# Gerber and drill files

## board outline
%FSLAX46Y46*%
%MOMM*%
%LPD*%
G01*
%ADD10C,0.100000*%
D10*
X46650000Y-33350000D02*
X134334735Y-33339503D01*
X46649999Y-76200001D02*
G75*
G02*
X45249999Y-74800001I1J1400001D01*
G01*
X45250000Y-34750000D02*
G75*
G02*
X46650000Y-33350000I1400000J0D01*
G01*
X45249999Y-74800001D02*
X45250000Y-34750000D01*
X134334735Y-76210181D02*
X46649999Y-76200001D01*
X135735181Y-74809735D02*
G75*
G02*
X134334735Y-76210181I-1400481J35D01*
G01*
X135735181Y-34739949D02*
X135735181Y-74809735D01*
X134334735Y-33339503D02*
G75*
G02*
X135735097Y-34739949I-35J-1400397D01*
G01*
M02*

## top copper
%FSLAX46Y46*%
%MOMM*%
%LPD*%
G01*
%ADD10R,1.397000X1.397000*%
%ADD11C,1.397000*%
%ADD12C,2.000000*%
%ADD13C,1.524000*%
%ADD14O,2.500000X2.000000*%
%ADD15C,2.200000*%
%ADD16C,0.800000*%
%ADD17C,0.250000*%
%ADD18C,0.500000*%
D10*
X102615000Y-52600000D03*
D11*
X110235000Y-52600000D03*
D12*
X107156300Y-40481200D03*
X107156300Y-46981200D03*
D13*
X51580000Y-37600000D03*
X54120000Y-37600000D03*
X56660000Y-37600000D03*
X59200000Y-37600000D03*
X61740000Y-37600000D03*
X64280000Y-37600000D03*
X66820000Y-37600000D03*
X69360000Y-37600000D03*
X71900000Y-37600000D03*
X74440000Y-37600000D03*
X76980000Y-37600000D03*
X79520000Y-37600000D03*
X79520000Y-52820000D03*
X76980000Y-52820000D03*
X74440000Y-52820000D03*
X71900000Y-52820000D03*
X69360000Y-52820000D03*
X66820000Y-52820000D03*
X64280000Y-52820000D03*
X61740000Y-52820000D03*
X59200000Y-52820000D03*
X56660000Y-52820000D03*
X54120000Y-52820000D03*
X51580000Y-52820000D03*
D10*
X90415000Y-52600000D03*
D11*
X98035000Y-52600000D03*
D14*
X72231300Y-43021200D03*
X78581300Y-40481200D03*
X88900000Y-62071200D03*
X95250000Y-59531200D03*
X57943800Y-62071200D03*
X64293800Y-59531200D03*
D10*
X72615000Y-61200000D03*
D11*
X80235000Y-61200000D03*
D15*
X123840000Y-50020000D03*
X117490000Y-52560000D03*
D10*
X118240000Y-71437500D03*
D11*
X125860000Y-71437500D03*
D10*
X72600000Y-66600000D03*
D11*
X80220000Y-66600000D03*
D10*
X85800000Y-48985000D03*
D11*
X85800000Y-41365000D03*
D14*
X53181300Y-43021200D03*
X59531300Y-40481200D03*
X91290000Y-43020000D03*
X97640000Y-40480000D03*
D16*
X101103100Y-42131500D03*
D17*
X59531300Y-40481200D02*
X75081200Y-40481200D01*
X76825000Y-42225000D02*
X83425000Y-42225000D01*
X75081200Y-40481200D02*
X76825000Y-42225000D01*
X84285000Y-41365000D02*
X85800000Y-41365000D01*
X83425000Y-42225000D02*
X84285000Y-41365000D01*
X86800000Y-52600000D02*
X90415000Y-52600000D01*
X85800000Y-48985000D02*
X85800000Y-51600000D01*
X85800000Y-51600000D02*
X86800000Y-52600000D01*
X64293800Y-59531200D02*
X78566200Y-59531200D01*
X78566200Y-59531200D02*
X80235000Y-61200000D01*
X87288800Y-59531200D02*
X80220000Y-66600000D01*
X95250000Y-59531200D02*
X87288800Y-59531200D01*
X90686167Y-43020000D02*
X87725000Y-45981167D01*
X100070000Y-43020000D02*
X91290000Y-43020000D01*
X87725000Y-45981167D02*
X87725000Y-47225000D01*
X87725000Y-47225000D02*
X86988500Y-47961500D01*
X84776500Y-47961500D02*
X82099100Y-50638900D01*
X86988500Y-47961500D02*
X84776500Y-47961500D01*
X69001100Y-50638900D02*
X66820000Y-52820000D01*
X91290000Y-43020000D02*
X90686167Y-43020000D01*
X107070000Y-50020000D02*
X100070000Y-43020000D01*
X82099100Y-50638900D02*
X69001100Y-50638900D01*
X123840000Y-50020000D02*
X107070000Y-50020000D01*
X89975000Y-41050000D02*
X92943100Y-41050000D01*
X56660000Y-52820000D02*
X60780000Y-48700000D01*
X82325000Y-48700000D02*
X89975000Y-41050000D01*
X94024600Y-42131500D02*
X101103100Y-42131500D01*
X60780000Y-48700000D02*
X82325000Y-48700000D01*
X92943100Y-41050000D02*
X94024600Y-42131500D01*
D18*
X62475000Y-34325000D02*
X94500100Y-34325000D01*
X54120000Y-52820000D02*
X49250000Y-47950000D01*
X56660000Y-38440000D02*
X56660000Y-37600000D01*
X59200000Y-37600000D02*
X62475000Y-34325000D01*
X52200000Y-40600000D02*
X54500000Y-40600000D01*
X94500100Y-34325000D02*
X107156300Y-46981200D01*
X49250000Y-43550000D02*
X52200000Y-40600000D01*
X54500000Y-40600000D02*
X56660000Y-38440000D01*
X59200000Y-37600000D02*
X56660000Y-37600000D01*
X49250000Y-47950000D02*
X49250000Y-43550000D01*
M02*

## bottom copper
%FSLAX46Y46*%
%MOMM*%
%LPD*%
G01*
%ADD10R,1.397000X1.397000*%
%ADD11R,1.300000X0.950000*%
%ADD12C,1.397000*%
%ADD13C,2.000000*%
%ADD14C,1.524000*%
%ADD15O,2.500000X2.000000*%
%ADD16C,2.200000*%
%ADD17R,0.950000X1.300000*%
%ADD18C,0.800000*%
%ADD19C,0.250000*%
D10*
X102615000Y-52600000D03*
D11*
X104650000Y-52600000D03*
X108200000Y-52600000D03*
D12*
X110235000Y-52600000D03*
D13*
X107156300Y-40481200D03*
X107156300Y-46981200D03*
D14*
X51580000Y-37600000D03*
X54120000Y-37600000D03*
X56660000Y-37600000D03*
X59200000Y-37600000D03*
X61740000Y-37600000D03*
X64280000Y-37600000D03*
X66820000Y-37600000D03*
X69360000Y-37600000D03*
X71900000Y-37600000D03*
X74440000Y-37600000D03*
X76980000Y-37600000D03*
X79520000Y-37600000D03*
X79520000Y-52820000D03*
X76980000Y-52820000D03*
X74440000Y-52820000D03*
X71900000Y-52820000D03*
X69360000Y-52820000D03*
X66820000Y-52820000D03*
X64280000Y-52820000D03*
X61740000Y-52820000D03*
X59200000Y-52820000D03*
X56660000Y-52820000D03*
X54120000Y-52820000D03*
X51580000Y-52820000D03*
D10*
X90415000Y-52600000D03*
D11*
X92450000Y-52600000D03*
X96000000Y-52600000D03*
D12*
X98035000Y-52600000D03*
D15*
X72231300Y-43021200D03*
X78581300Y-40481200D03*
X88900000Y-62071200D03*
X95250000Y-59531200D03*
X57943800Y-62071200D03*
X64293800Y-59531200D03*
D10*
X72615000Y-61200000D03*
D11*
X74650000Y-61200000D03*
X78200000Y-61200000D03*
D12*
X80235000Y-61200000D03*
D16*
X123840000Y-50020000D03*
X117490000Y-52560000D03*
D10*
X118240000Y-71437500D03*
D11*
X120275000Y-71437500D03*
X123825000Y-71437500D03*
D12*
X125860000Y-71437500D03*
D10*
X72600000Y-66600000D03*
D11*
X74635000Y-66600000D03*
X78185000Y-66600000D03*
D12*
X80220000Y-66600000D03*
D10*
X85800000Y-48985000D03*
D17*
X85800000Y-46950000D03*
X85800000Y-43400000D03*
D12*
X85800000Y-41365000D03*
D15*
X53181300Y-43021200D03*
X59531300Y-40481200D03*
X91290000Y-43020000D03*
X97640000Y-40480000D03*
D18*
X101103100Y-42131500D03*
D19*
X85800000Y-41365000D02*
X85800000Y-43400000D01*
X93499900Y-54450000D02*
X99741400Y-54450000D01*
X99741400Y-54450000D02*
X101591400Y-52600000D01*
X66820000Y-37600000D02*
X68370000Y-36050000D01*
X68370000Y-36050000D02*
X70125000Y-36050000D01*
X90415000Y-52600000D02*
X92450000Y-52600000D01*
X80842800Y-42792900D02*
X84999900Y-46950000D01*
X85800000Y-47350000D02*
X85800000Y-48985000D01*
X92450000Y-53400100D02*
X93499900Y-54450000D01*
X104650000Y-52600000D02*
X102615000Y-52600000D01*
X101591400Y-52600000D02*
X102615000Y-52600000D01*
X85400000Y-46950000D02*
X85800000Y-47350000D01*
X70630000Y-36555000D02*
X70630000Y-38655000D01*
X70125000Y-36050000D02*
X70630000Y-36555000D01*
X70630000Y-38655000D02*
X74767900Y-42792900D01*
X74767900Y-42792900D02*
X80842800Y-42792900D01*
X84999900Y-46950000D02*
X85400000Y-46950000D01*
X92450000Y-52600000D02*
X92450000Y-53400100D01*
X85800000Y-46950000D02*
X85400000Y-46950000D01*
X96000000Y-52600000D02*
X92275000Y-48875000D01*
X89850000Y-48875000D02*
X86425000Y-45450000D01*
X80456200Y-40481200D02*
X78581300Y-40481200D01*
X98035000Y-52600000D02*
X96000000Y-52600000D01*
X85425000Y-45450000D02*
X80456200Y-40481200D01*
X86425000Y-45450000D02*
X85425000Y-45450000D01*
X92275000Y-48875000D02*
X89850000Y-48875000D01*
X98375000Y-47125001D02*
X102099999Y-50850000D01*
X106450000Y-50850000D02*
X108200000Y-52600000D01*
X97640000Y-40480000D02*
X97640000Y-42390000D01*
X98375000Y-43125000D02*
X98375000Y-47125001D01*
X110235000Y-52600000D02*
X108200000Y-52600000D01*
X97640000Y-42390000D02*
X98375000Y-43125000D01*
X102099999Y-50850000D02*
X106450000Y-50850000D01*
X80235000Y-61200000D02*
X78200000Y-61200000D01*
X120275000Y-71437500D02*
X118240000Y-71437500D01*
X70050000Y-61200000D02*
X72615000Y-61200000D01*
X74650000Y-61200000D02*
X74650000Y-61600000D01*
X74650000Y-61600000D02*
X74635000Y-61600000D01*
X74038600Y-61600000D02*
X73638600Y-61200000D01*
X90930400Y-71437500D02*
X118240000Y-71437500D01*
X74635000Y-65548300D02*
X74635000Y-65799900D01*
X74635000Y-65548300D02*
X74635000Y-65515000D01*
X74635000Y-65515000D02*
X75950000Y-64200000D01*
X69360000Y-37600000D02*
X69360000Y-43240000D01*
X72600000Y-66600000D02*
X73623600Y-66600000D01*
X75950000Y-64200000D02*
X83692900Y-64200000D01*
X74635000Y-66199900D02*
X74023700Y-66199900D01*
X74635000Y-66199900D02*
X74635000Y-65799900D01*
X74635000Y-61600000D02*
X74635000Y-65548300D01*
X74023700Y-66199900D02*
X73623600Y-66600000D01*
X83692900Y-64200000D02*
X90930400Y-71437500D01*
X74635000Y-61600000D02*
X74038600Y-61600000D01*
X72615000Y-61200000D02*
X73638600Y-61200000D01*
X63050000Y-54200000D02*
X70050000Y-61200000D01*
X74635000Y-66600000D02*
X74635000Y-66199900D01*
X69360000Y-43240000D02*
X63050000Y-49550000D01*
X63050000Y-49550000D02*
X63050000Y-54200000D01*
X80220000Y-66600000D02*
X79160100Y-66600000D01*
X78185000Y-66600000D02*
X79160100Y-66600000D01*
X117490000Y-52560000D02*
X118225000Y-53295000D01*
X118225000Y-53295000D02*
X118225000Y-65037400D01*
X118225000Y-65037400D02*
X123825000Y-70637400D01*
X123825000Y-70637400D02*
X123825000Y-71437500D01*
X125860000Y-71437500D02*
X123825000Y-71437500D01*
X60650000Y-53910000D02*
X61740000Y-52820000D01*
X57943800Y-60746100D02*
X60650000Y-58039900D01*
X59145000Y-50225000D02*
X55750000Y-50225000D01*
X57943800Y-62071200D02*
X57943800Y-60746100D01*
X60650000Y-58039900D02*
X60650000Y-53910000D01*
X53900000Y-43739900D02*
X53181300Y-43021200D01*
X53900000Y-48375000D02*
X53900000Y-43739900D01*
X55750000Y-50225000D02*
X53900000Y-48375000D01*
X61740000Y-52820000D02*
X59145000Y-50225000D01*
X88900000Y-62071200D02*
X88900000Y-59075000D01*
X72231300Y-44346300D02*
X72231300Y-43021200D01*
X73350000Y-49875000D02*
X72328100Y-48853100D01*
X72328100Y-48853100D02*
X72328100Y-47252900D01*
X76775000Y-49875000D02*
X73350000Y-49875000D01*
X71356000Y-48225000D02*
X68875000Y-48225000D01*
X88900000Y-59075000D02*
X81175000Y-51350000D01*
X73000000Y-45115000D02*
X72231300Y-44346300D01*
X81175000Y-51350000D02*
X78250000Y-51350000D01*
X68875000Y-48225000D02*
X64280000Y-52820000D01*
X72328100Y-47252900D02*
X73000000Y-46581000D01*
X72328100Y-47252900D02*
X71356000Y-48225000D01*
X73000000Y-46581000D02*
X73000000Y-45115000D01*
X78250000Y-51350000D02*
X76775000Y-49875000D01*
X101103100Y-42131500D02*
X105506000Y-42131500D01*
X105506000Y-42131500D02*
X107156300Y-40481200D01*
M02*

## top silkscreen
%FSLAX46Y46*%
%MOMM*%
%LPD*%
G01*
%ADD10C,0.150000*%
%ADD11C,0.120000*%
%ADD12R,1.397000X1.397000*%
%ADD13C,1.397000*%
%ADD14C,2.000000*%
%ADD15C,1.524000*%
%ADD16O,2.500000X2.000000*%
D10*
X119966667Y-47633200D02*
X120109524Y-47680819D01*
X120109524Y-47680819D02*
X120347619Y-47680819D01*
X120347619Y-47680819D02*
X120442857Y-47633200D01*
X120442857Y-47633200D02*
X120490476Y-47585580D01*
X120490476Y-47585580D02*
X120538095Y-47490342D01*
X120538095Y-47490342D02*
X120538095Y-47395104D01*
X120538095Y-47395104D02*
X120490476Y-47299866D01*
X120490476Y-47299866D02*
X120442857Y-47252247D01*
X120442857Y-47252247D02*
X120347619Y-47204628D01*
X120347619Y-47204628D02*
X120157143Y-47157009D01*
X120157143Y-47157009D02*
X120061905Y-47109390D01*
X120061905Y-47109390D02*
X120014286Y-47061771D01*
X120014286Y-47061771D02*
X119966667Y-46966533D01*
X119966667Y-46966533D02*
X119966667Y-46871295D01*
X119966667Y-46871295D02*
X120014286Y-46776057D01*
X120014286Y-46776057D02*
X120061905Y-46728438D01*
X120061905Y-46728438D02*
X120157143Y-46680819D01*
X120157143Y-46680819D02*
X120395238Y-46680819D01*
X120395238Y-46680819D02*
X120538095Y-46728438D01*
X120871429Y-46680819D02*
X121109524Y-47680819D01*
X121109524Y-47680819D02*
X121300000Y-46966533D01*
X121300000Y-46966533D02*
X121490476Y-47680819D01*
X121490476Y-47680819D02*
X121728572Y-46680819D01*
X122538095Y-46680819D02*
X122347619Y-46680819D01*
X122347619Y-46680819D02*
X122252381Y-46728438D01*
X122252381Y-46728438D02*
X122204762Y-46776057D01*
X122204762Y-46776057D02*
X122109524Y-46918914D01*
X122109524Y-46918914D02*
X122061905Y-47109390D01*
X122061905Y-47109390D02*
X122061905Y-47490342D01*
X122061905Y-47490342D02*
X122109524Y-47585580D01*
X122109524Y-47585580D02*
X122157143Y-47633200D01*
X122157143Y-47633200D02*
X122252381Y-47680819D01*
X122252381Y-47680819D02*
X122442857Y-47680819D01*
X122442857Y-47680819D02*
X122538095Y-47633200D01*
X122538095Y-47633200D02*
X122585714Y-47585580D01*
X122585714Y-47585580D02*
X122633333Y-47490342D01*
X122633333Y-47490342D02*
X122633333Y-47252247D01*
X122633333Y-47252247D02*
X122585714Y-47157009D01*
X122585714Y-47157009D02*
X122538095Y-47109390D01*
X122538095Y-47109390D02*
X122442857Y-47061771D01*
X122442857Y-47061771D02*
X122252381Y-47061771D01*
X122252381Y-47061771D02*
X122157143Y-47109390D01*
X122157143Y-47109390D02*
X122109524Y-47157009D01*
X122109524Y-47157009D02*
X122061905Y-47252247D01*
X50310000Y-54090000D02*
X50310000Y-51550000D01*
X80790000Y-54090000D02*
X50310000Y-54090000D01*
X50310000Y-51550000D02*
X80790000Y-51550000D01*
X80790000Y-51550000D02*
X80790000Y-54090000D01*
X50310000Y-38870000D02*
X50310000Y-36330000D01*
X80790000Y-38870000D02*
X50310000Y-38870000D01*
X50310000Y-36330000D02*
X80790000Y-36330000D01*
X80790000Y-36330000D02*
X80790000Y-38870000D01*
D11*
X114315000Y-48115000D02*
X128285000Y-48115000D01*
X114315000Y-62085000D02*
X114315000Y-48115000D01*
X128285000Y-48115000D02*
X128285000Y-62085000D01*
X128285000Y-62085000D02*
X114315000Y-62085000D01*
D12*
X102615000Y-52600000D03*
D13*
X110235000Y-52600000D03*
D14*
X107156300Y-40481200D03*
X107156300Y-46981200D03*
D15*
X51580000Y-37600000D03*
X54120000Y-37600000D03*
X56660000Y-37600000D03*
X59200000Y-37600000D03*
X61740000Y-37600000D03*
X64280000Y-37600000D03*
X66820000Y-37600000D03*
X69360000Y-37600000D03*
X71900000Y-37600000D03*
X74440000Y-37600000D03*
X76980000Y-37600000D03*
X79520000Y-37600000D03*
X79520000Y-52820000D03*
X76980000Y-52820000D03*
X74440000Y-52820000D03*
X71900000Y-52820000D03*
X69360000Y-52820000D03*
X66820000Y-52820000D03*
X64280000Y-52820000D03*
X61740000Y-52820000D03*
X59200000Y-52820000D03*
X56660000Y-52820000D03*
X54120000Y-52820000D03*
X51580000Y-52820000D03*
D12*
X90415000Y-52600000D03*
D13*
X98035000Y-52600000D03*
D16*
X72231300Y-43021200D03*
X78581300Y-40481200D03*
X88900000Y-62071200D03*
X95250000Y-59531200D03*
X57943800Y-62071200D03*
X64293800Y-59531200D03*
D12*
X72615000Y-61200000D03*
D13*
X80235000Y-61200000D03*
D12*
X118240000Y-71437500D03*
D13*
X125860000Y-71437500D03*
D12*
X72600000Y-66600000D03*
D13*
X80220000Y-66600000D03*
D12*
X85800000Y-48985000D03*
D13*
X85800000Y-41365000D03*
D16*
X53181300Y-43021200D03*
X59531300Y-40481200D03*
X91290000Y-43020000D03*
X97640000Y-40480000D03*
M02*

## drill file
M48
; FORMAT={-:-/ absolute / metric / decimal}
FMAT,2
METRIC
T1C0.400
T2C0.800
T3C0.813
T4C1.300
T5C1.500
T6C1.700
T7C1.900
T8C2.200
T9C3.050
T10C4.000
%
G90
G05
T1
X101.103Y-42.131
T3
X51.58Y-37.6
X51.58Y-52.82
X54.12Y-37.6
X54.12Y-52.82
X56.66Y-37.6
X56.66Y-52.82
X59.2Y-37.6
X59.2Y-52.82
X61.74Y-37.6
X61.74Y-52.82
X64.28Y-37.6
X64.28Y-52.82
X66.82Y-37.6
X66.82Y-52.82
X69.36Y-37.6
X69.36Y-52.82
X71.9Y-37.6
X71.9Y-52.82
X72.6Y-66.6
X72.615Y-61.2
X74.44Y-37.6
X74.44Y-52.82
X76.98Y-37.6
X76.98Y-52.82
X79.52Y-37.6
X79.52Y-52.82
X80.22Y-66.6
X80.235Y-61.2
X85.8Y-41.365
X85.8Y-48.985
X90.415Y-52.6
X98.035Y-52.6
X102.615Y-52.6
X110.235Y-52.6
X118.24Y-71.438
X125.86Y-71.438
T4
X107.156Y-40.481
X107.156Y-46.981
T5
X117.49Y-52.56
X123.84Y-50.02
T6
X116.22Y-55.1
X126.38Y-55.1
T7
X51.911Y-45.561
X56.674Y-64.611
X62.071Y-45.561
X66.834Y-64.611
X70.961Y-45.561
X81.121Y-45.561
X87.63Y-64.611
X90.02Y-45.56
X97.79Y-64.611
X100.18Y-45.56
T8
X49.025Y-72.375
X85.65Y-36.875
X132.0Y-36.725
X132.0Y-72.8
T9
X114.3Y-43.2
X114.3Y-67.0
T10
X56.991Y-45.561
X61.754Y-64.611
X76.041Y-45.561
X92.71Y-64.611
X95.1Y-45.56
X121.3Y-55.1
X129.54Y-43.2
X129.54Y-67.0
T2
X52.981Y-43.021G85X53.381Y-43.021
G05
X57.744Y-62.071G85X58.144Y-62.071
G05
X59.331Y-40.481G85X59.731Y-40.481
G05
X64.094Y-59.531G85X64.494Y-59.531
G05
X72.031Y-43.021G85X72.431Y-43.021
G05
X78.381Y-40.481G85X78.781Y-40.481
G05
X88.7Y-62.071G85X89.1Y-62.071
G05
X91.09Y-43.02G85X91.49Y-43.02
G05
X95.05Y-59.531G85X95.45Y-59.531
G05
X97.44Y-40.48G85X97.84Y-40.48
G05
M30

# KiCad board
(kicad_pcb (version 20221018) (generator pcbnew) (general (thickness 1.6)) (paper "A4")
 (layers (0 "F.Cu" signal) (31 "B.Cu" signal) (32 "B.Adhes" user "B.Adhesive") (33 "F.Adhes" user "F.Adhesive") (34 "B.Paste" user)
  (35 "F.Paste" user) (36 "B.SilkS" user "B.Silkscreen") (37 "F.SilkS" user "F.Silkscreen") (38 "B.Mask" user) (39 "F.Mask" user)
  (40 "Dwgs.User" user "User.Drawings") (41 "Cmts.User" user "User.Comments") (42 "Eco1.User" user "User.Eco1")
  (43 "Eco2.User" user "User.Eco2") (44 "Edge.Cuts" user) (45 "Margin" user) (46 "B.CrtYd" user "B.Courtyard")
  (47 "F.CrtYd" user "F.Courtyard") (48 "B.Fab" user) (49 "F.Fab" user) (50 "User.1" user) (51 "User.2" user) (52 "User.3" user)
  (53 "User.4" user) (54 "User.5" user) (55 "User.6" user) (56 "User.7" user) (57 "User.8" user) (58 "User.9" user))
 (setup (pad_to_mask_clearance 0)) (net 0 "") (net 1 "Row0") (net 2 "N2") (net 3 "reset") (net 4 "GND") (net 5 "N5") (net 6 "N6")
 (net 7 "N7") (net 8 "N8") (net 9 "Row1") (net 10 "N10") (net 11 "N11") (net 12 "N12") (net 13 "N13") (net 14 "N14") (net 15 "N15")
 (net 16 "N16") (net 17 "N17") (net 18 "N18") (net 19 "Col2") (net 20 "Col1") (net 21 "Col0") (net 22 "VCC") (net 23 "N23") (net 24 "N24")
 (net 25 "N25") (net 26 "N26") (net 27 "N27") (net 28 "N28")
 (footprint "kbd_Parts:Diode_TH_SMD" (layer "F.Cu") (at 106.425 52.6)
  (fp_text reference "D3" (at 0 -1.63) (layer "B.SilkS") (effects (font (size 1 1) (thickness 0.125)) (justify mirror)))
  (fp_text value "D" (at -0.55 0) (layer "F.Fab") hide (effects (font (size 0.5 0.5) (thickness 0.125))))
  (pad "1" thru_hole rect (at -3.81 0) (size 1.397 1.397) (drill 0.8128) (layers "*.Cu" "*.Mask" "F.SilkS") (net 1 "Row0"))
  (pad "1" smd rect (at -1.775 0) (size 1.3 0.95) (layers "B.Cu" "B.Paste" "B.Mask") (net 1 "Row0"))
  (pad "2" smd rect (at 1.775 0) (size 1.3 0.95) (layers "B.Cu" "B.Paste" "B.Mask") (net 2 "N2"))
  (pad "2" thru_hole circle (at 3.81 0) (size 1.397 1.397) (drill 0.8128) (layers "*.Cu" "*.Mask" "F.SilkS") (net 2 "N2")))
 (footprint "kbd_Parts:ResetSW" (layer "F.Cu") (at 107.1563 43.7312 90)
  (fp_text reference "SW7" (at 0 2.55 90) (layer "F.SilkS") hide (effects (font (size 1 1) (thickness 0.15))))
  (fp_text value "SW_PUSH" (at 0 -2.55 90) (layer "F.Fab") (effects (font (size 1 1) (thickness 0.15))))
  (pad "1" thru_hole circle (at 3.25 0 90) (size 2 2) (drill 1.3) (layers "*.Cu" "*.Mask" "F.SilkS") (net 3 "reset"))
  (pad "2" thru_hole circle (at -3.25 0 90) (size 2 2) (drill 1.3) (layers "*.Cu" "*.Mask" "F.SilkS") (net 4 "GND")))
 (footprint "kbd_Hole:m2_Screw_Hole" (layer "F.Cu") (at 85.65 36.875)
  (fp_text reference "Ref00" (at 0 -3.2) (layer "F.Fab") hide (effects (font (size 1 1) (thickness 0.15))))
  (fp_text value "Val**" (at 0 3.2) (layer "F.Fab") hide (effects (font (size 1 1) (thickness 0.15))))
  (pad "" np_thru_hole circle (at 0 0) (size 2.2 2.2) (drill 2.2) (layers "*.Cu" "*.Mask")))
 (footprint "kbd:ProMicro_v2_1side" (layer "F.Cu") (at 66.058 45.2564 90)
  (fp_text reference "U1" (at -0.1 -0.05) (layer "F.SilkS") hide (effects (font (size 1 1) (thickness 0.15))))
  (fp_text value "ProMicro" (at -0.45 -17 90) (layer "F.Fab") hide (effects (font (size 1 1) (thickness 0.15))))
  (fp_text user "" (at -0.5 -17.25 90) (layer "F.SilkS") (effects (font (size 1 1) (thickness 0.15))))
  (fp_line (start -8.8336 -15.748) (end -6.2936 -15.748) (stroke (width 0.15) (type solid)) (layer "F.SilkS"))
  (fp_line (start -8.8336 14.732) (end -8.8336 -15.748) (stroke (width 0.15) (type solid)) (layer "F.SilkS"))
  (fp_line (start -6.2936 -15.748) (end -6.2936 14.732) (stroke (width 0.15) (type solid)) (layer "F.SilkS"))
  (fp_line (start -6.2936 14.732) (end -8.8336 14.732) (stroke (width 0.15) (type solid)) (layer "F.SilkS"))
  (fp_line (start 6.3864 -15.748) (end 8.9264 -15.748) (stroke (width 0.15) (type solid)) (layer "F.SilkS"))
  (fp_line (start 6.3864 14.732) (end 6.3864 -15.748) (stroke (width 0.15) (type solid)) (layer "F.SilkS"))
  (fp_line (start 8.9264 -15.748) (end 8.9264 14.732) (stroke (width 0.15) (type solid)) (layer "F.SilkS"))
  (fp_line (start 8.9264 14.732) (end 6.3864 14.732) (stroke (width 0.15) (type solid)) (layer "F.SilkS"))
  (pad "1" thru_hole circle (at 7.6564 -14.478 90) (size 1.524 1.524) (drill 0.8128) (layers "*.Cu" "F.SilkS" "B.Mask") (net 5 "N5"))
  (pad "2" thru_hole circle (at 7.6564 -11.938 90) (size 1.524 1.524) (drill 0.8128) (layers "*.Cu" "F.SilkS" "B.Mask") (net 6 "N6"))
  (pad "3" thru_hole circle (at 7.6564 -9.398 90) (size 1.524 1.524) (drill 0.8128) (layers "*.Cu" "F.SilkS" "B.Mask") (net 4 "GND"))
  (pad "4" thru_hole circle (at 7.6564 -6.858 90) (size 1.524 1.524) (drill 0.8128) (layers "*.Cu" "F.SilkS" "B.Mask") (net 4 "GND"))
  (pad "5" thru_hole circle (at 7.6564 -4.318 90) (size 1.524 1.524) (drill 0.8128) (layers "*.Cu" "F.SilkS" "B.Mask") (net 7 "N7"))
  (pad "6" thru_hole circle (at 7.6564 -1.778 90) (size 1.524 1.524) (drill 0.8128) (layers "*.Cu" "F.SilkS" "B.Mask") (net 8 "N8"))
  (pad "7" thru_hole circle (at 7.6564 0.762 90) (size 1.524 1.524) (drill 0.8128) (layers "*.Cu" "F.SilkS" "B.Mask") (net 1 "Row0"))
  (pad "8" thru_hole circle (at 7.6564 3.302 90) (size 1.524 1.524) (drill 0.8128) (layers "*.Cu" "F.SilkS" "B.Mask") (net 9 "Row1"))
  (pad "9" thru_hole circle (at 7.6564 5.842 90) (size 1.524 1.524) (drill 0.8128) (layers "*.Cu" "F.SilkS" "B.Mask") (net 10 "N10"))
  (pad "10" thru_hole circle (at 7.6564 8.382 90) (size 1.524 1.524) (drill 0.8128) (layers "*.Cu" "F.SilkS" "B.Mask") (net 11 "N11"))
  (pad "11" thru_hole circle (at 7.6564 10.922 90) (size 1.524 1.524) (drill 0.8128) (layers "*.Cu" "F.SilkS" "B.Mask") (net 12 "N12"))
  (pad "12" thru_hole circle (at 7.6564 13.462 90) (size 1.524 1.524) (drill 0.8128) (layers "*.Cu" "F.SilkS" "B.Mask") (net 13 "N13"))
  (pad "13" thru_hole circle (at -7.5636 13.462 90) (size 1.524 1.524) (drill 0.8128) (layers "*.Cu" "F.SilkS" "B.Mask") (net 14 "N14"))
  (pad "14" thru_hole circle (at -7.5636 10.922 90) (size 1.524 1.524) (drill 0.8128) (layers "*.Cu" "F.SilkS" "B.Mask") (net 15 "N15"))
  (pad "15" thru_hole circle (at -7.5636 8.382 90) (size 1.524 1.524) (drill 0.8128) (layers "*.Cu" "F.SilkS" "B.Mask") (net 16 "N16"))
  (pad "16" thru_hole circle (at -7.5636 5.842 90) (size 1.524 1.524) (drill 0.8128) (layers "*.Cu" "F.SilkS" "B.Mask") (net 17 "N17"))
  (pad "17" thru_hole circle (at -7.5636 3.302 90) (size 1.524 1.524) (drill 0.8128) (layers "*.Cu" "F.SilkS" "B.Mask") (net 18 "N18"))
  (pad "18" thru_hole circle (at -7.5636 0.762 90) (size 1.524 1.524) (drill 0.8128) (layers "*.Cu" "F.SilkS" "B.Mask") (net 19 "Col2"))
  (pad "19" thru_hole circle (at -7.5636 -1.778 90) (size 1.524 1.524) (drill 0.8128) (layers "*.Cu" "F.SilkS" "B.Mask") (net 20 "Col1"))
  (pad "20" thru_hole circle (at -7.5636 -4.318 90) (size 1.524 1.524) (drill 0.8128) (layers "*.Cu" "F.SilkS" "B.Mask") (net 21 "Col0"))
  (pad "21" thru_hole circle (at -7.5636 -6.858 90) (size 1.524 1.524) (drill 0.8128) (layers "*.Cu" "F.SilkS" "B.Mask") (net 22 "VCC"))
  (pad "22" thru_hole circle (at -7.5636 -9.398 90) (size 1.524 1.524) (drill 0.8128) (layers "*.Cu" "F.SilkS" "B.Mask") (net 3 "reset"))
  (pad "23" thru_hole circle (at -7.5636 -11.938 90) (size 1.524 1.524) (drill 0.8128) (layers "*.Cu" "F.SilkS" "B.Mask") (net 4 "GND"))
  (pad "24" thru_hole circle (at -7.5636 -14.478 90) (size 1.524 1.524) (drill 0.8128) (layers "*.Cu" "F.SilkS" "B.Mask") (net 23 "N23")))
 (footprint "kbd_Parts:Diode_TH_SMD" (layer "F.Cu") (at 94.225 52.6)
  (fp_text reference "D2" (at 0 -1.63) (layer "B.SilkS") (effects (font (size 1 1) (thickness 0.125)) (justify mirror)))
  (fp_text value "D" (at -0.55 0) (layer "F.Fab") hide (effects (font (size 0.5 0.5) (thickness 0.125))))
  (pad "1" thru_hole rect (at -3.81 0) (size 1.397 1.397) (drill 0.8128) (layers "*.Cu" "*.Mask" "F.SilkS") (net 1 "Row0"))
  (pad "1" smd rect (at -1.775 0) (size 1.3 0.95) (layers "B.Cu" "B.Paste" "B.Mask") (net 1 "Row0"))
  (pad "2" smd rect (at 1.775 0) (size 1.3 0.95) (layers "B.Cu" "B.Paste" "B.Mask") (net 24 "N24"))
  (pad "2" thru_hole circle (at 3.81 0) (size 1.397 1.397) (drill 0.8128) (layers "*.Cu" "*.Mask" "F.SilkS") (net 24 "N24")))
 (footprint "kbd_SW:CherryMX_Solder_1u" (layer "F.Cu") (at 76.0413 45.5612)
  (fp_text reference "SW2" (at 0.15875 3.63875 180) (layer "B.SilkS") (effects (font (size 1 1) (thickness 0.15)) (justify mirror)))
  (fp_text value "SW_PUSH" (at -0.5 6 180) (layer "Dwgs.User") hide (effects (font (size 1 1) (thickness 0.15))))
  (pad "" np_thru_hole circle (at -5.08 0 90) (size 1.9 1.9) (drill 1.9) (layers "*.Cu" "*.Mask"))
  (pad "" np_thru_hole circle (at 0 0 90) (size 4 4) (drill 4) (layers "*.Cu" "*.Mask"))
  (pad "" np_thru_hole circle (at 5.08 0 90) (size 1.9 1.9) (drill 1.9) (layers "*.Cu" "*.Mask"))
  (pad "1" thru_hole oval (at -3.81 -2.54) (size 2.5 2) (drill oval 1.2 0.8) (layers "*.Cu" "F.SilkS" "B.Mask") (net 20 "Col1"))
  (pad "2" thru_hole oval (at 2.54 -5.08) (size 2.5 2) (drill oval 1.2 0.8) (layers "*.Cu" "F.SilkS" "B.Mask") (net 24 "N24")))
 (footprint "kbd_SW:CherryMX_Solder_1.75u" (layer "F.Cu") (at 92.71 64.6112)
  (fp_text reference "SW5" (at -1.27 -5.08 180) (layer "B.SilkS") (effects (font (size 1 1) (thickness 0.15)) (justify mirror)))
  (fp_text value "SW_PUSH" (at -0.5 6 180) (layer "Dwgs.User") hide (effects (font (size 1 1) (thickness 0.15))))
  (pad "" np_thru_hole circle (at -5.08 0 90) (size 1.9 1.9) (drill 1.9) (layers "*.Cu" "*.Mask"))
  (pad "" np_thru_hole circle (at 0 0 90) (size 4 4) (drill 4) (layers "*.Cu" "*.Mask"))
  (pad "" np_thru_hole circle (at 5.08 0 90) (size 1.9 1.9) (drill 1.9) (layers "*.Cu" "*.Mask"))
  (pad "1" thru_hole oval (at -3.81 -2.54) (size 2.5 2) (drill oval 1.2 0.8) (layers "*.Cu" "F.SilkS" "B.Mask") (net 20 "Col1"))
  (pad "2" thru_hole oval (at 2.54 -5.08) (size 2.5 2) (drill oval 1.2 0.8) (layers "*.Cu" "F.SilkS" "B.Mask") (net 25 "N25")))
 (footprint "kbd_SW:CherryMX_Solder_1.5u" (layer "F.Cu") (at 61.7538 64.6112)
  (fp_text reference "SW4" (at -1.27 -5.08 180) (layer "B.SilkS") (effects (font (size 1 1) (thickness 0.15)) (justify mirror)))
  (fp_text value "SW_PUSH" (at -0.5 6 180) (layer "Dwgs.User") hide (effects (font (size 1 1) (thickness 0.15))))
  (pad "" np_thru_hole circle (at -5.08 0 90) (size 1.9 1.9) (drill 1.9) (layers "*.Cu" "*.Mask"))
  (pad "" np_thru_hole circle (at 0 0 90) (size 4 4) (drill 4) (layers "*.Cu" "*.Mask"))
  (pad "" np_thru_hole circle (at 5.08 0 90) (size 1.9 1.9) (drill 1.9) (layers "*.Cu" "*.Mask"))
  (pad "1" thru_hole oval (at -3.81 -2.54) (size 2.5 2) (drill oval 1.2 0.8) (layers "*.Cu" "F.SilkS" "B.Mask") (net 21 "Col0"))
  (pad "2" thru_hole oval (at 2.54 -5.08) (size 2.5 2) (drill oval 1.2 0.8) (layers "*.Cu" "F.SilkS" "B.Mask") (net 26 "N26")))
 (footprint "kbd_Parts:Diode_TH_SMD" (layer "F.Cu") (at 76.425 61.2)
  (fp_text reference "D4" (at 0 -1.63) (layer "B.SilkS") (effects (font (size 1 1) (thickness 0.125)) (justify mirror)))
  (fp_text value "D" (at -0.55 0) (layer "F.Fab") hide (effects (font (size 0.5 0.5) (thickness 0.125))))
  (pad "1" thru_hole rect (at -3.81 0) (size 1.397 1.397) (drill 0.8128) (layers "*.Cu" "*.Mask" "F.SilkS") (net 9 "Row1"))
  (pad "1" smd rect (at -1.775 0) (size 1.3 0.95) (layers "B.Cu" "B.Paste" "B.Mask") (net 9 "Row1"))
  (pad "2" smd rect (at 1.775 0) (size 1.3 0.95) (layers "B.Cu" "B.Paste" "B.Mask") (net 26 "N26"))
  (pad "2" thru_hole circle (at 3.81 0) (size 1.397 1.397) (drill 0.8128) (layers "*.Cu" "*.Mask" "F.SilkS") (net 26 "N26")))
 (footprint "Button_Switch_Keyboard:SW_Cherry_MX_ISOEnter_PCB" (layer "F.Cu") (at 123.84 50.02)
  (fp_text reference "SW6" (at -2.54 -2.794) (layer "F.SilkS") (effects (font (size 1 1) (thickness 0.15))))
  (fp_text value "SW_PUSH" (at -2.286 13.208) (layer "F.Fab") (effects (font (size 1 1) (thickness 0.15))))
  (fp_line (start -9.525 -1.905) (end 4.445 -1.905) (stroke (width 0.12) (type solid)) (layer "F.SilkS"))
  (fp_line (start -9.525 12.065) (end -9.525 -1.905) (stroke (width 0.12) (type solid)) (layer "F.SilkS"))
  (fp_line (start 4.445 -1.905) (end 4.445 12.065) (stroke (width 0.12) (type solid)) (layer "F.SilkS"))
  (fp_line (start 4.445 12.065) (end -9.525 12.065) (stroke (width 0.12) (type solid)) (layer "F.SilkS"))
  (pad "" np_thru_hole circle (at -9.54 -6.82) (size 3.05 3.05) (drill 3.05) (layers "*.Cu" "*.Mask"))
  (pad "" np_thru_hole circle (at -9.54 16.98) (size 3.05 3.05) (drill 3.05) (layers "*.Cu" "*.Mask"))
  (pad "" np_thru_hole circle (at -7.62 5.08) (size 1.7 1.7) (drill 1.7) (layers "*.Cu" "*.Mask"))
  (pad "" np_thru_hole circle (at -2.54 5.08) (size 4 4) (drill 4) (layers "*.Cu" "*.Mask"))
  (pad "" np_thru_hole circle (at 2.54 5.08) (size 1.7 1.7) (drill 1.7) (layers "*.Cu" "*.Mask"))
  (pad "" np_thru_hole circle (at 5.7 -6.82) (size 4 4) (drill 4) (layers "*.Cu" "*.Mask"))
  (pad "" np_thru_hole circle (at 5.7 16.98) (size 4 4) (drill 4) (layers "*.Cu" "*.Mask"))
  (pad "1" thru_hole circle (at 0 0) (size 2.2 2.2) (drill 1.5) (layers "*.Cu" "*.Mask") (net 19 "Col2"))
  (pad "2" thru_hole circle (at -6.35 2.54) (size 2.2 2.2) (drill 1.5) (layers "*.Cu" "*.Mask") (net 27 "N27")))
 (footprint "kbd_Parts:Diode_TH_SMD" (layer "F.Cu") (at 122.05 71.4375)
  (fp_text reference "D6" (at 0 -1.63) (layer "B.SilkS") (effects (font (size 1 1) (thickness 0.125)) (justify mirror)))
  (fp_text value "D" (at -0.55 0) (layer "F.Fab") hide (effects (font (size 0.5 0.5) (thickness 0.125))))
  (pad "1" thru_hole rect (at -3.81 0) (size 1.397 1.397) (drill 0.8128) (layers "*.Cu" "*.Mask" "F.SilkS") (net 9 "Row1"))
  (pad "1" smd rect (at -1.775 0) (size 1.3 0.95) (layers "B.Cu" "B.Paste" "B.Mask") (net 9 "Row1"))
  (pad "2" smd rect (at 1.775 0) (size 1.3 0.95) (layers "B.Cu" "B.Paste" "B.Mask") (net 27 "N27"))
  (pad "2" thru_hole circle (at 3.81 0) (size 1.397 1.397) (drill 0.8128) (layers "*.Cu" "*.Mask" "F.SilkS") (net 27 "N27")))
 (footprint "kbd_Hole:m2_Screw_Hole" (layer "F.Cu") (at 132 36.725)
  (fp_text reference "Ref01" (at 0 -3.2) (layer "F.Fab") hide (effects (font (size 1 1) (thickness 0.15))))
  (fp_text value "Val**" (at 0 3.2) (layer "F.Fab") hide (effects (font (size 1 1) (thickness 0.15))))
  (pad "" np_thru_hole circle (at 0 0) (size 2.2 2.2) (drill 2.2) (layers "*.Cu" "*.Mask")))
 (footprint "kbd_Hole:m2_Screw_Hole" (layer "F.Cu") (at 132 72.8)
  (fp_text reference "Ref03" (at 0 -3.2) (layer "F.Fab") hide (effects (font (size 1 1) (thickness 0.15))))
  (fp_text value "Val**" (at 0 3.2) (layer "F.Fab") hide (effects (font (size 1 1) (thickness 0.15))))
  (pad "" np_thru_hole circle (at 0 0) (size 2.2 2.2) (drill 2.2) (layers "*.Cu" "*.Mask")))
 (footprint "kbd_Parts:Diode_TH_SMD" (layer "F.Cu") (at 76.41 66.6)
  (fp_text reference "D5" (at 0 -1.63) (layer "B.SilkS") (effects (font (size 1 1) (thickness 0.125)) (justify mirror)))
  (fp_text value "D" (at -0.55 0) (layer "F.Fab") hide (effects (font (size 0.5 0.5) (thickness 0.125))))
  (pad "1" thru_hole rect (at -3.81 0) (size 1.397 1.397) (drill 0.8128) (layers "*.Cu" "*.Mask" "F.SilkS") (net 9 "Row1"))
  (pad "1" smd rect (at -1.775 0) (size 1.3 0.95) (layers "B.Cu" "B.Paste" "B.Mask") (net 9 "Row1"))
  (pad "2" smd rect (at 1.775 0) (size 1.3 0.95) (layers "B.Cu" "B.Paste" "B.Mask") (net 25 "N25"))
  (pad "2" thru_hole circle (at 3.81 0) (size 1.397 1.397) (drill 0.8128) (layers "*.Cu" "*.Mask" "F.SilkS") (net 25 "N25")))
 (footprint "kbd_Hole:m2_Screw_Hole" (layer "F.Cu") (at 49.025 72.375)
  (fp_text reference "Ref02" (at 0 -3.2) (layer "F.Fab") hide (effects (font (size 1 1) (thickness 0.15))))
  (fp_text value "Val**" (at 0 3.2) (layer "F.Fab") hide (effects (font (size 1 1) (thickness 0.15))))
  (pad "" np_thru_hole circle (at 0 0) (size 2.2 2.2) (drill 2.2) (layers "*.Cu" "*.Mask")))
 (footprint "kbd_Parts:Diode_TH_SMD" (layer "F.Cu") (at 85.8 45.175 90)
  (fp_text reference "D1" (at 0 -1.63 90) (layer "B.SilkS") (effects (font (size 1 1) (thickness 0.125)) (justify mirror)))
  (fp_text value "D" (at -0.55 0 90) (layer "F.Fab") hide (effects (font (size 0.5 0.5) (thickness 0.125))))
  (pad "1" thru_hole rect (at -3.81 0 90) (size 1.397 1.397) (drill 0.8128) (layers "*.Cu" "*.Mask" "F.SilkS") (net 1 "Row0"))
  (pad "1" smd rect (at -1.775 0 90) (size 1.3 0.95) (layers "B.Cu" "B.Paste" "B.Mask") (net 1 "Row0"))
  (pad "2" smd rect (at 1.775 0 90) (size 1.3 0.95) (layers "B.Cu" "B.Paste" "B.Mask") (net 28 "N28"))
  (pad "2" thru_hole circle (at 3.81 0 90) (size 1.397 1.397) (drill 0.8128) (layers "*.Cu" "*.Mask" "F.SilkS") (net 28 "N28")))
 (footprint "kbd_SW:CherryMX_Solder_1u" (layer "F.Cu") (at 56.9913 45.5612)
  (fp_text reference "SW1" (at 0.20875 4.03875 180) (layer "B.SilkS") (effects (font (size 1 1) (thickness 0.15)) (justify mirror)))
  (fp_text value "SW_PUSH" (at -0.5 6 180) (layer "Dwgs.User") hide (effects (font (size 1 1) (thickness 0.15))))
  (pad "" np_thru_hole circle (at -5.08 0 90) (size 1.9 1.9) (drill 1.9) (layers "*.Cu" "*.Mask"))
  (pad "" np_thru_hole circle (at 0 0 90) (size 4 4) (drill 4) (layers "*.Cu" "*.Mask"))
  (pad "" np_thru_hole circle (at 5.08 0 90) (size 1.9 1.9) (drill 1.9) (layers "*.Cu" "*.Mask"))
  (pad "1" thru_hole oval (at -3.81 -2.54) (size 2.5 2) (drill oval 1.2 0.8) (layers "*.Cu" "F.SilkS" "B.Mask") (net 21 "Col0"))
  (pad "2" thru_hole oval (at 2.54 -5.08) (size 2.5 2) (drill oval 1.2 0.8) (layers "*.Cu" "F.SilkS" "B.Mask") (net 28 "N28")))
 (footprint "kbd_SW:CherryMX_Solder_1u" (layer "F.Cu") (at 95.1 45.56)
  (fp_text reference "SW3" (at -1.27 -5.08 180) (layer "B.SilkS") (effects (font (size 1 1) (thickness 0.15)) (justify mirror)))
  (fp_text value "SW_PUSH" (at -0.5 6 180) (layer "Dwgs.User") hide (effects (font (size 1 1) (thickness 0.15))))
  (pad "" np_thru_hole circle (at -5.08 0 90) (size 1.9 1.9) (drill 1.9) (layers "*.Cu" "*.Mask"))
  (pad "" np_thru_hole circle (at 0 0 90) (size 4 4) (drill 4) (layers "*.Cu" "*.Mask"))
  (pad "" np_thru_hole circle (at 5.08 0 90) (size 1.9 1.9) (drill 1.9) (layers "*.Cu" "*.Mask"))
  (pad "1" thru_hole oval (at -3.81 -2.54) (size 2.5 2) (drill oval 1.2 0.8) (layers "*.Cu" "F.SilkS" "B.Mask") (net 19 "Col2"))
  (pad "2" thru_hole oval (at 2.54 -5.08) (size 2.5 2) (drill oval 1.2 0.8) (layers "*.Cu" "F.SilkS" "B.Mask") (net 2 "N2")))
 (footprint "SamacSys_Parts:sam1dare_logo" (layer "B.Cu") (at 105.4 69.4 180)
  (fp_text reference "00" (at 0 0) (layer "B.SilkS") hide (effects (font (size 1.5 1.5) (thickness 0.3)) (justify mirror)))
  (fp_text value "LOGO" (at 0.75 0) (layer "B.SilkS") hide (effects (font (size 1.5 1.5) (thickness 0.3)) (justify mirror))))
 (gr_line (start 46.65 33.35) (end 134.334735 33.339503) (stroke (width 0.1) (type default)) (layer "Edge.Cuts"))
 (gr_arc (start 46.649999 76.200001) (mid 45.66005 75.78995) (end 45.249999 74.800001) (stroke (width 0.1) (type default))
  (layer "Edge.Cuts"))
 (gr_arc (start 45.25 34.75) (mid 45.660051 33.760051) (end 46.65 33.35) (stroke (width 0.1) (type default)) (layer "Edge.Cuts"))
 (gr_line (start 45.249999 74.800001) (end 45.25 34.75) (stroke (width 0.1) (type default)) (layer "Edge.Cuts"))
 (gr_line (start 134.334735 76.210181) (end 46.649999 76.200001) (stroke (width 0.1) (type default)) (layer "Edge.Cuts"))
 (gr_arc (start 135.735181 74.809735) (mid 135.325 75.8) (end 134.334735 76.210181) (stroke (width 0.1) (type default)) (layer "Edge.Cuts"))
 (gr_line (start 135.735181 34.739949) (end 135.735181 74.809735) (stroke (width 0.1) (type default)) (layer "Edge.Cuts"))
 (gr_arc (start 134.334735 33.339503) (mid 135.325 33.749684) (end 135.735181 34.739949) (stroke (width 0.1) (type default))
  (layer "Edge.Cuts"))
 (segment (start 59.5313 40.4812) (end 75.0812 40.4812) (width 0.25) (layer "F.Cu") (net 28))
 (segment (start 76.825 42.225) (end 83.425 42.225) (width 0.25) (layer "F.Cu") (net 28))
 (segment (start 75.0812 40.4812) (end 76.825 42.225) (width 0.25) (layer "F.Cu") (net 28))
 (segment (start 84.285 41.365) (end 85.8 41.365) (width 0.25) (layer "F.Cu") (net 28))
 (segment (start 83.425 42.225) (end 84.285 41.365) (width 0.25) (layer "F.Cu") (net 28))
 (segment (start 85.8 41.365) (end 85.8 43.4) (width 0.25) (layer "B.Cu") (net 28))
 (segment (start 86.8 52.6) (end 90.415 52.6) (width 0.25) (layer "F.Cu") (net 1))
 (segment (start 85.8 48.985) (end 85.8 51.6) (width 0.25) (layer "F.Cu") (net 1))
 (segment (start 85.8 51.6) (end 86.8 52.6) (width 0.25) (layer "F.Cu") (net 1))
 (segment (start 93.4999 54.45) (end 99.7414 54.45) (width 0.25) (layer "B.Cu") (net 1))
 (segment (start 99.7414 54.45) (end 101.5914 52.6) (width 0.25) (layer "B.Cu") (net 1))
 (segment (start 66.82 37.6) (end 68.37 36.05) (width 0.25) (layer "B.Cu") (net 1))
 (segment (start 68.37 36.05) (end 70.125 36.05) (width 0.25) (layer "B.Cu") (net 1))
 (segment (start 90.415 52.6) (end 92.45 52.6) (width 0.25) (layer "B.Cu") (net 1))
 (segment (start 80.8428 42.7929) (end 84.9999 46.95) (width 0.25) (layer "B.Cu") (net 1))
 (segment (start 85.8 47.35) (end 85.8 48.985) (width 0.25) (layer "B.Cu") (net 1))
 (segment (start 92.45 53.4001) (end 93.4999 54.45) (width 0.25) (layer "B.Cu") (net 1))
 (segment (start 104.65 52.6) (end 102.615 52.6) (width 0.25) (layer "B.Cu") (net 1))
 (segment (start 101.5914 52.6) (end 102.615 52.6) (width 0.25) (layer "B.Cu") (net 1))
 (segment (start 85.4 46.95) (end 85.8 47.35) (width 0.25) (layer "B.Cu") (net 1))
 (segment (start 70.63 36.555) (end 70.63 38.655) (width 0.25) (layer "B.Cu") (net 1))
 (segment (start 70.125 36.05) (end 70.63 36.555) (width 0.25) (layer "B.Cu") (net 1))
 (segment (start 70.63 38.655) (end 74.7679 42.7929) (width 0.25) (layer "B.Cu") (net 1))
 (segment (start 74.7679 42.7929) (end 80.8428 42.7929) (width 0.25) (layer "B.Cu") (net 1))
 (segment (start 84.9999 46.95) (end 85.4 46.95) (width 0.25) (layer "B.Cu") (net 1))
 (segment (start 92.45 52.6) (end 92.45 53.4001) (width 0.25) (layer "B.Cu") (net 1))
 (segment (start 85.8 46.95) (end 85.4 46.95) (width 0.25) (layer "B.Cu") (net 1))
 (segment (start 96 52.6) (end 92.275 48.875) (width 0.25) (layer "B.Cu") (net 24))
 (segment (start 89.85 48.875) (end 86.425 45.45) (width 0.25) (layer "B.Cu") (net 24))
 (segment (start 80.4562 40.4812) (end 78.5813 40.4812) (width 0.25) (layer "B.Cu") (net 24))
 (segment (start 98.035 52.6) (end 96 52.6) (width 0.25) (layer "B.Cu") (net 24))
 (segment (start 85.425 45.45) (end 80.4562 40.4812) (width 0.25) (layer "B.Cu") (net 24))
 (segment (start 86.425 45.45) (end 85.425 45.45) (width 0.25) (layer "B.Cu") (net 24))
 (segment (start 92.275 48.875) (end 89.85 48.875) (width 0.25) (layer "B.Cu") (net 24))
 (segment (start 98.375 47.125001) (end 102.099999 50.85) (width 0.25) (layer "B.Cu") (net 2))
 (segment (start 106.45 50.85) (end 108.2 52.6) (width 0.25) (layer "B.Cu") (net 2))
 (segment (start 97.64 40.48) (end 97.64 42.39) (width 0.25) (layer "B.Cu") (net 2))
 (segment (start 98.375 43.125) (end 98.375 47.125001) (width 0.25) (layer "B.Cu") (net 2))
 (segment (start 110.235 52.6) (end 108.2 52.6) (width 0.25) (layer "B.Cu") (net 2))
 (segment (start 97.64 42.39) (end 98.375 43.125) (width 0.25) (layer "B.Cu") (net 2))
 (segment (start 102.099999 50.85) (end 106.45 50.85) (width 0.25) (layer "B.Cu") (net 2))
 (segment (start 64.2938 59.5312) (end 78.5662 59.5312) (width 0.25) (layer "F.Cu") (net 26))
 (segment (start 78.5662 59.5312) (end 80.235 61.2) (width 0.25) (layer "F.Cu") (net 26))
 (segment (start 80.235 61.2) (end 78.2 61.2) (width 0.25) (layer "B.Cu") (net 26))
 (segment (start 120.275 71.4375) (end 118.24 71.4375) (width 0.25) (layer "B.Cu") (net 9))
 (segment (start 70.05 61.2) (end 72.615 61.2) (width 0.25) (layer "B.Cu") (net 9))
 (segment (start 74.65 61.2) (end 74.65 61.6) (width 0.25) (layer "B.Cu") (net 9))
 (segment (start 74.65 61.6) (end 74.635 61.6) (width 0.25) (layer "B.Cu") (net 9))
 (segment (start 74.0386 61.6) (end 73.6386 61.2) (width 0.25) (layer "B.Cu") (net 9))
 (segment (start 90.9304 71.4375) (end 118.24 71.4375) (width 0.25) (layer "B.Cu") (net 9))
 (segment (start 74.635 65.5483) (end 74.635 65.7999) (width 0.25) (layer "B.Cu") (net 9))
 (segment (start 74.635 65.5483) (end 74.635 65.515) (width 0.25) (layer "B.Cu") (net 9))
 (segment (start 74.635 65.515) (end 75.95 64.2) (width 0.25) (layer "B.Cu") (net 9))
 (segment (start 69.36 37.6) (end 69.36 43.24) (width 0.25) (layer "B.Cu") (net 9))
 (segment (start 72.6 66.6) (end 73.6236 66.6) (width 0.25) (layer "B.Cu") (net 9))
 (segment (start 75.95 64.2) (end 83.6929 64.2) (width 0.25) (layer "B.Cu") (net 9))
 (segment (start 74.635 66.1999) (end 74.0237 66.1999) (width 0.25) (layer "B.Cu") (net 9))
 (segment (start 74.635 66.1999) (end 74.635 65.7999) (width 0.25) (layer "B.Cu") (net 9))
 (segment (start 74.635 61.6) (end 74.635 65.5483) (width 0.25) (layer "B.Cu") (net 9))
 (segment (start 74.0237 66.1999) (end 73.6236 66.6) (width 0.25) (layer "B.Cu") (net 9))
 (segment (start 83.6929 64.2) (end 90.9304 71.4375) (width 0.25) (layer "B.Cu") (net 9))
 (segment (start 74.635 61.6) (end 74.0386 61.6) (width 0.25) (layer "B.Cu") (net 9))
 (segment (start 72.615 61.2) (end 73.6386 61.2) (width 0.25) (layer "B.Cu") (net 9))
 (segment (start 63.05 54.2) (end 70.05 61.2) (width 0.25) (layer "B.Cu") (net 9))
 (segment (start 74.635 66.6) (end 74.635 66.1999) (width 0.25) (layer "B.Cu") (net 9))
 (segment (start 69.36 43.24) (end 63.05 49.55) (width 0.25) (layer "B.Cu") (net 9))
 (segment (start 63.05 49.55) (end 63.05 54.2) (width 0.25) (layer "B.Cu") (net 9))
 (segment (start 87.2888 59.5312) (end 80.22 66.6) (width 0.25) (layer "F.Cu") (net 25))
 (segment (start 95.25 59.5312) (end 87.2888 59.5312) (width 0.25) (layer "F.Cu") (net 25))
 (segment (start 80.22 66.6) (end 79.1601 66.6) (width 0.25) (layer "B.Cu") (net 25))
 (segment (start 78.185 66.6) (end 79.1601 66.6) (width 0.25) (layer "B.Cu") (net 25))
 (segment (start 117.49 52.56) (end 118.225 53.295) (width 0.25) (layer "B.Cu") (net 27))
 (segment (start 118.225 53.295) (end 118.225 65.0374) (width 0.25) (layer "B.Cu") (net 27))
 (segment (start 118.225 65.0374) (end 123.825 70.6374) (width 0.25) (layer "B.Cu") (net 27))
 (segment (start 123.825 70.6374) (end 123.825 71.4375) (width 0.25) (layer "B.Cu") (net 27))
 (segment (start 125.86 71.4375) (end 123.825 71.4375) (width 0.25) (layer "B.Cu") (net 27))
 (segment (start 60.65 53.91) (end 61.74 52.82) (width 0.25) (layer "B.Cu") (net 21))
 (segment (start 57.9438 60.7461) (end 60.65 58.0399) (width 0.25) (layer "B.Cu") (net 21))
 (segment (start 59.145 50.225) (end 55.75 50.225) (width 0.25) (layer "B.Cu") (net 21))
 (segment (start 57.9438 62.0712) (end 57.9438 60.7461) (width 0.25) (layer "B.Cu") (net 21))
 (segment (start 60.65 58.0399) (end 60.65 53.91) (width 0.25) (layer "B.Cu") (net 21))
 (segment (start 53.9 43.7399) (end 53.1813 43.0212) (width 0.25) (layer "B.Cu") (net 21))
 (segment (start 53.9 48.375) (end 53.9 43.7399) (width 0.25) (layer "B.Cu") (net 21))
 (segment (start 55.75 50.225) (end 53.9 48.375) (width 0.25) (layer "B.Cu") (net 21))
 (segment (start 61.74 52.82) (end 59.145 50.225) (width 0.25) (layer "B.Cu") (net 21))
 (segment (start 88.9 62.0712) (end 88.9 59.075) (width 0.25) (layer "B.Cu") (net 20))
 (segment (start 72.2313 44.3463) (end 72.2313 43.0212) (width 0.25) (layer "B.Cu") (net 20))
 (segment (start 73.35 49.875) (end 72.3281 48.8531) (width 0.25) (layer "B.Cu") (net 20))
 (segment (start 72.3281 48.8531) (end 72.3281 47.2529) (width 0.25) (layer "B.Cu") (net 20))
 (segment (start 76.775 49.875) (end 73.35 49.875) (width 0.25) (layer "B.Cu") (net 20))
 (segment (start 71.356 48.225) (end 68.875 48.225) (width 0.25) (layer "B.Cu") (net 20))
 (segment (start 88.9 59.075) (end 81.175 51.35) (width 0.25) (layer "B.Cu") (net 20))
 (segment (start 73 45.115) (end 72.2313 44.3463) (width 0.25) (layer "B.Cu") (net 20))
 (segment (start 81.175 51.35) (end 78.25 51.35) (width 0.25) (layer "B.Cu") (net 20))
 (segment (start 68.875 48.225) (end 64.28 52.82) (width 0.25) (layer "B.Cu") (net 20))
 (segment (start 72.3281 47.2529) (end 73 46.581) (width 0.25) (layer "B.Cu") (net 20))
 (segment (start 72.3281 47.2529) (end 71.356 48.225) (width 0.25) (layer "B.Cu") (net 20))
 (segment (start 73 46.581) (end 73 45.115) (width 0.25) (layer "B.Cu") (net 20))
 (segment (start 78.25 51.35) (end 76.775 49.875) (width 0.25) (layer "B.Cu") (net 20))
 (segment (start 90.686167 43.02) (end 87.725 45.981167) (width 0.25) (layer "F.Cu") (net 19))
 (segment (start 100.07 43.02) (end 91.29 43.02) (width 0.25) (layer "F.Cu") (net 19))
 (segment (start 87.725 45.981167) (end 87.725 47.225) (width 0.25) (layer "F.Cu") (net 19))
 (segment (start 87.725 47.225) (end 86.9885 47.9615) (width 0.25) (layer "F.Cu") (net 19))
 (segment (start 84.7765 47.9615) (end 82.0991 50.6389) (width 0.25) (layer "F.Cu") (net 19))
 (segment (start 86.9885 47.9615) (end 84.7765 47.9615) (width 0.25) (layer "F.Cu") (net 19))
 (segment (start 69.0011 50.6389) (end 66.82 52.82) (width 0.25) (layer "F.Cu") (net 19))
 (segment (start 91.29 43.02) (end 90.686167 43.02) (width 0.25) (layer "F.Cu") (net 19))
 (segment (start 107.07 50.02) (end 100.07 43.02) (width 0.25) (layer "F.Cu") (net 19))
 (segment (start 82.0991 50.6389) (end 69.0011 50.6389) (width 0.25) (layer "F.Cu") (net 19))
 (segment (start 123.84 50.02) (end 107.07 50.02) (width 0.25) (layer "F.Cu") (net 19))
 (segment (start 89.975 41.05) (end 92.9431 41.05) (width 0.25) (layer "F.Cu") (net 3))
 (segment (start 56.66 52.82) (end 60.78 48.7) (width 0.25) (layer "F.Cu") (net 3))
 (segment (start 82.325 48.7) (end 89.975 41.05) (width 0.25) (layer "F.Cu") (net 3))
 (segment (start 94.0246 42.1315) (end 101.1031 42.1315) (width 0.25) (layer "F.Cu") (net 3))
 (segment (start 60.78 48.7) (end 82.325 48.7) (width 0.25) (layer "F.Cu") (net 3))
 (segment (start 92.9431 41.05) (end 94.0246 42.1315) (width 0.25) (layer "F.Cu") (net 3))
 (via (at 101.1031 42.1315) (size 0.8) (drill 0.4) (layers "F.Cu" "B.Cu") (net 3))
 (segment (start 101.1031 42.1315) (end 105.506 42.1315) (width 0.25) (layer "B.Cu") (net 3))
 (segment (start 105.506 42.1315) (end 107.1563 40.4812) (width 0.25) (layer "B.Cu") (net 3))
 (segment (start 62.475 34.325) (end 94.5001 34.325) (width 0.5) (layer "F.Cu") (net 4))
 (segment (start 54.12 52.82) (end 49.25 47.95) (width 0.5) (layer "F.Cu") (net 4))
 (segment (start 56.66 38.44) (end 56.66 37.6) (width 0.5) (layer "F.Cu") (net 4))
 (segment (start 59.2 37.6) (end 62.475 34.325) (width 0.5) (layer "F.Cu") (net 4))
 (segment (start 52.2 40.6) (end 54.5 40.6) (width 0.5) (layer "F.Cu") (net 4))
 (segment (start 94.5001 34.325) (end 107.1563 46.9812) (width 0.5) (layer "F.Cu") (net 4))
 (segment (start 49.25 43.55) (end 52.2 40.6) (width 0.5) (layer "F.Cu") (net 4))
 (segment (start 54.5 40.6) (end 56.66 38.44) (width 0.5) (layer "F.Cu") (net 4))
 (segment (start 59.2 37.6) (end 56.66 37.6) (width 0.5) (layer "F.Cu") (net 4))
 (segment (start 49.25 47.95) (end 49.25 43.55) (width 0.5) (layer "F.Cu") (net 4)))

